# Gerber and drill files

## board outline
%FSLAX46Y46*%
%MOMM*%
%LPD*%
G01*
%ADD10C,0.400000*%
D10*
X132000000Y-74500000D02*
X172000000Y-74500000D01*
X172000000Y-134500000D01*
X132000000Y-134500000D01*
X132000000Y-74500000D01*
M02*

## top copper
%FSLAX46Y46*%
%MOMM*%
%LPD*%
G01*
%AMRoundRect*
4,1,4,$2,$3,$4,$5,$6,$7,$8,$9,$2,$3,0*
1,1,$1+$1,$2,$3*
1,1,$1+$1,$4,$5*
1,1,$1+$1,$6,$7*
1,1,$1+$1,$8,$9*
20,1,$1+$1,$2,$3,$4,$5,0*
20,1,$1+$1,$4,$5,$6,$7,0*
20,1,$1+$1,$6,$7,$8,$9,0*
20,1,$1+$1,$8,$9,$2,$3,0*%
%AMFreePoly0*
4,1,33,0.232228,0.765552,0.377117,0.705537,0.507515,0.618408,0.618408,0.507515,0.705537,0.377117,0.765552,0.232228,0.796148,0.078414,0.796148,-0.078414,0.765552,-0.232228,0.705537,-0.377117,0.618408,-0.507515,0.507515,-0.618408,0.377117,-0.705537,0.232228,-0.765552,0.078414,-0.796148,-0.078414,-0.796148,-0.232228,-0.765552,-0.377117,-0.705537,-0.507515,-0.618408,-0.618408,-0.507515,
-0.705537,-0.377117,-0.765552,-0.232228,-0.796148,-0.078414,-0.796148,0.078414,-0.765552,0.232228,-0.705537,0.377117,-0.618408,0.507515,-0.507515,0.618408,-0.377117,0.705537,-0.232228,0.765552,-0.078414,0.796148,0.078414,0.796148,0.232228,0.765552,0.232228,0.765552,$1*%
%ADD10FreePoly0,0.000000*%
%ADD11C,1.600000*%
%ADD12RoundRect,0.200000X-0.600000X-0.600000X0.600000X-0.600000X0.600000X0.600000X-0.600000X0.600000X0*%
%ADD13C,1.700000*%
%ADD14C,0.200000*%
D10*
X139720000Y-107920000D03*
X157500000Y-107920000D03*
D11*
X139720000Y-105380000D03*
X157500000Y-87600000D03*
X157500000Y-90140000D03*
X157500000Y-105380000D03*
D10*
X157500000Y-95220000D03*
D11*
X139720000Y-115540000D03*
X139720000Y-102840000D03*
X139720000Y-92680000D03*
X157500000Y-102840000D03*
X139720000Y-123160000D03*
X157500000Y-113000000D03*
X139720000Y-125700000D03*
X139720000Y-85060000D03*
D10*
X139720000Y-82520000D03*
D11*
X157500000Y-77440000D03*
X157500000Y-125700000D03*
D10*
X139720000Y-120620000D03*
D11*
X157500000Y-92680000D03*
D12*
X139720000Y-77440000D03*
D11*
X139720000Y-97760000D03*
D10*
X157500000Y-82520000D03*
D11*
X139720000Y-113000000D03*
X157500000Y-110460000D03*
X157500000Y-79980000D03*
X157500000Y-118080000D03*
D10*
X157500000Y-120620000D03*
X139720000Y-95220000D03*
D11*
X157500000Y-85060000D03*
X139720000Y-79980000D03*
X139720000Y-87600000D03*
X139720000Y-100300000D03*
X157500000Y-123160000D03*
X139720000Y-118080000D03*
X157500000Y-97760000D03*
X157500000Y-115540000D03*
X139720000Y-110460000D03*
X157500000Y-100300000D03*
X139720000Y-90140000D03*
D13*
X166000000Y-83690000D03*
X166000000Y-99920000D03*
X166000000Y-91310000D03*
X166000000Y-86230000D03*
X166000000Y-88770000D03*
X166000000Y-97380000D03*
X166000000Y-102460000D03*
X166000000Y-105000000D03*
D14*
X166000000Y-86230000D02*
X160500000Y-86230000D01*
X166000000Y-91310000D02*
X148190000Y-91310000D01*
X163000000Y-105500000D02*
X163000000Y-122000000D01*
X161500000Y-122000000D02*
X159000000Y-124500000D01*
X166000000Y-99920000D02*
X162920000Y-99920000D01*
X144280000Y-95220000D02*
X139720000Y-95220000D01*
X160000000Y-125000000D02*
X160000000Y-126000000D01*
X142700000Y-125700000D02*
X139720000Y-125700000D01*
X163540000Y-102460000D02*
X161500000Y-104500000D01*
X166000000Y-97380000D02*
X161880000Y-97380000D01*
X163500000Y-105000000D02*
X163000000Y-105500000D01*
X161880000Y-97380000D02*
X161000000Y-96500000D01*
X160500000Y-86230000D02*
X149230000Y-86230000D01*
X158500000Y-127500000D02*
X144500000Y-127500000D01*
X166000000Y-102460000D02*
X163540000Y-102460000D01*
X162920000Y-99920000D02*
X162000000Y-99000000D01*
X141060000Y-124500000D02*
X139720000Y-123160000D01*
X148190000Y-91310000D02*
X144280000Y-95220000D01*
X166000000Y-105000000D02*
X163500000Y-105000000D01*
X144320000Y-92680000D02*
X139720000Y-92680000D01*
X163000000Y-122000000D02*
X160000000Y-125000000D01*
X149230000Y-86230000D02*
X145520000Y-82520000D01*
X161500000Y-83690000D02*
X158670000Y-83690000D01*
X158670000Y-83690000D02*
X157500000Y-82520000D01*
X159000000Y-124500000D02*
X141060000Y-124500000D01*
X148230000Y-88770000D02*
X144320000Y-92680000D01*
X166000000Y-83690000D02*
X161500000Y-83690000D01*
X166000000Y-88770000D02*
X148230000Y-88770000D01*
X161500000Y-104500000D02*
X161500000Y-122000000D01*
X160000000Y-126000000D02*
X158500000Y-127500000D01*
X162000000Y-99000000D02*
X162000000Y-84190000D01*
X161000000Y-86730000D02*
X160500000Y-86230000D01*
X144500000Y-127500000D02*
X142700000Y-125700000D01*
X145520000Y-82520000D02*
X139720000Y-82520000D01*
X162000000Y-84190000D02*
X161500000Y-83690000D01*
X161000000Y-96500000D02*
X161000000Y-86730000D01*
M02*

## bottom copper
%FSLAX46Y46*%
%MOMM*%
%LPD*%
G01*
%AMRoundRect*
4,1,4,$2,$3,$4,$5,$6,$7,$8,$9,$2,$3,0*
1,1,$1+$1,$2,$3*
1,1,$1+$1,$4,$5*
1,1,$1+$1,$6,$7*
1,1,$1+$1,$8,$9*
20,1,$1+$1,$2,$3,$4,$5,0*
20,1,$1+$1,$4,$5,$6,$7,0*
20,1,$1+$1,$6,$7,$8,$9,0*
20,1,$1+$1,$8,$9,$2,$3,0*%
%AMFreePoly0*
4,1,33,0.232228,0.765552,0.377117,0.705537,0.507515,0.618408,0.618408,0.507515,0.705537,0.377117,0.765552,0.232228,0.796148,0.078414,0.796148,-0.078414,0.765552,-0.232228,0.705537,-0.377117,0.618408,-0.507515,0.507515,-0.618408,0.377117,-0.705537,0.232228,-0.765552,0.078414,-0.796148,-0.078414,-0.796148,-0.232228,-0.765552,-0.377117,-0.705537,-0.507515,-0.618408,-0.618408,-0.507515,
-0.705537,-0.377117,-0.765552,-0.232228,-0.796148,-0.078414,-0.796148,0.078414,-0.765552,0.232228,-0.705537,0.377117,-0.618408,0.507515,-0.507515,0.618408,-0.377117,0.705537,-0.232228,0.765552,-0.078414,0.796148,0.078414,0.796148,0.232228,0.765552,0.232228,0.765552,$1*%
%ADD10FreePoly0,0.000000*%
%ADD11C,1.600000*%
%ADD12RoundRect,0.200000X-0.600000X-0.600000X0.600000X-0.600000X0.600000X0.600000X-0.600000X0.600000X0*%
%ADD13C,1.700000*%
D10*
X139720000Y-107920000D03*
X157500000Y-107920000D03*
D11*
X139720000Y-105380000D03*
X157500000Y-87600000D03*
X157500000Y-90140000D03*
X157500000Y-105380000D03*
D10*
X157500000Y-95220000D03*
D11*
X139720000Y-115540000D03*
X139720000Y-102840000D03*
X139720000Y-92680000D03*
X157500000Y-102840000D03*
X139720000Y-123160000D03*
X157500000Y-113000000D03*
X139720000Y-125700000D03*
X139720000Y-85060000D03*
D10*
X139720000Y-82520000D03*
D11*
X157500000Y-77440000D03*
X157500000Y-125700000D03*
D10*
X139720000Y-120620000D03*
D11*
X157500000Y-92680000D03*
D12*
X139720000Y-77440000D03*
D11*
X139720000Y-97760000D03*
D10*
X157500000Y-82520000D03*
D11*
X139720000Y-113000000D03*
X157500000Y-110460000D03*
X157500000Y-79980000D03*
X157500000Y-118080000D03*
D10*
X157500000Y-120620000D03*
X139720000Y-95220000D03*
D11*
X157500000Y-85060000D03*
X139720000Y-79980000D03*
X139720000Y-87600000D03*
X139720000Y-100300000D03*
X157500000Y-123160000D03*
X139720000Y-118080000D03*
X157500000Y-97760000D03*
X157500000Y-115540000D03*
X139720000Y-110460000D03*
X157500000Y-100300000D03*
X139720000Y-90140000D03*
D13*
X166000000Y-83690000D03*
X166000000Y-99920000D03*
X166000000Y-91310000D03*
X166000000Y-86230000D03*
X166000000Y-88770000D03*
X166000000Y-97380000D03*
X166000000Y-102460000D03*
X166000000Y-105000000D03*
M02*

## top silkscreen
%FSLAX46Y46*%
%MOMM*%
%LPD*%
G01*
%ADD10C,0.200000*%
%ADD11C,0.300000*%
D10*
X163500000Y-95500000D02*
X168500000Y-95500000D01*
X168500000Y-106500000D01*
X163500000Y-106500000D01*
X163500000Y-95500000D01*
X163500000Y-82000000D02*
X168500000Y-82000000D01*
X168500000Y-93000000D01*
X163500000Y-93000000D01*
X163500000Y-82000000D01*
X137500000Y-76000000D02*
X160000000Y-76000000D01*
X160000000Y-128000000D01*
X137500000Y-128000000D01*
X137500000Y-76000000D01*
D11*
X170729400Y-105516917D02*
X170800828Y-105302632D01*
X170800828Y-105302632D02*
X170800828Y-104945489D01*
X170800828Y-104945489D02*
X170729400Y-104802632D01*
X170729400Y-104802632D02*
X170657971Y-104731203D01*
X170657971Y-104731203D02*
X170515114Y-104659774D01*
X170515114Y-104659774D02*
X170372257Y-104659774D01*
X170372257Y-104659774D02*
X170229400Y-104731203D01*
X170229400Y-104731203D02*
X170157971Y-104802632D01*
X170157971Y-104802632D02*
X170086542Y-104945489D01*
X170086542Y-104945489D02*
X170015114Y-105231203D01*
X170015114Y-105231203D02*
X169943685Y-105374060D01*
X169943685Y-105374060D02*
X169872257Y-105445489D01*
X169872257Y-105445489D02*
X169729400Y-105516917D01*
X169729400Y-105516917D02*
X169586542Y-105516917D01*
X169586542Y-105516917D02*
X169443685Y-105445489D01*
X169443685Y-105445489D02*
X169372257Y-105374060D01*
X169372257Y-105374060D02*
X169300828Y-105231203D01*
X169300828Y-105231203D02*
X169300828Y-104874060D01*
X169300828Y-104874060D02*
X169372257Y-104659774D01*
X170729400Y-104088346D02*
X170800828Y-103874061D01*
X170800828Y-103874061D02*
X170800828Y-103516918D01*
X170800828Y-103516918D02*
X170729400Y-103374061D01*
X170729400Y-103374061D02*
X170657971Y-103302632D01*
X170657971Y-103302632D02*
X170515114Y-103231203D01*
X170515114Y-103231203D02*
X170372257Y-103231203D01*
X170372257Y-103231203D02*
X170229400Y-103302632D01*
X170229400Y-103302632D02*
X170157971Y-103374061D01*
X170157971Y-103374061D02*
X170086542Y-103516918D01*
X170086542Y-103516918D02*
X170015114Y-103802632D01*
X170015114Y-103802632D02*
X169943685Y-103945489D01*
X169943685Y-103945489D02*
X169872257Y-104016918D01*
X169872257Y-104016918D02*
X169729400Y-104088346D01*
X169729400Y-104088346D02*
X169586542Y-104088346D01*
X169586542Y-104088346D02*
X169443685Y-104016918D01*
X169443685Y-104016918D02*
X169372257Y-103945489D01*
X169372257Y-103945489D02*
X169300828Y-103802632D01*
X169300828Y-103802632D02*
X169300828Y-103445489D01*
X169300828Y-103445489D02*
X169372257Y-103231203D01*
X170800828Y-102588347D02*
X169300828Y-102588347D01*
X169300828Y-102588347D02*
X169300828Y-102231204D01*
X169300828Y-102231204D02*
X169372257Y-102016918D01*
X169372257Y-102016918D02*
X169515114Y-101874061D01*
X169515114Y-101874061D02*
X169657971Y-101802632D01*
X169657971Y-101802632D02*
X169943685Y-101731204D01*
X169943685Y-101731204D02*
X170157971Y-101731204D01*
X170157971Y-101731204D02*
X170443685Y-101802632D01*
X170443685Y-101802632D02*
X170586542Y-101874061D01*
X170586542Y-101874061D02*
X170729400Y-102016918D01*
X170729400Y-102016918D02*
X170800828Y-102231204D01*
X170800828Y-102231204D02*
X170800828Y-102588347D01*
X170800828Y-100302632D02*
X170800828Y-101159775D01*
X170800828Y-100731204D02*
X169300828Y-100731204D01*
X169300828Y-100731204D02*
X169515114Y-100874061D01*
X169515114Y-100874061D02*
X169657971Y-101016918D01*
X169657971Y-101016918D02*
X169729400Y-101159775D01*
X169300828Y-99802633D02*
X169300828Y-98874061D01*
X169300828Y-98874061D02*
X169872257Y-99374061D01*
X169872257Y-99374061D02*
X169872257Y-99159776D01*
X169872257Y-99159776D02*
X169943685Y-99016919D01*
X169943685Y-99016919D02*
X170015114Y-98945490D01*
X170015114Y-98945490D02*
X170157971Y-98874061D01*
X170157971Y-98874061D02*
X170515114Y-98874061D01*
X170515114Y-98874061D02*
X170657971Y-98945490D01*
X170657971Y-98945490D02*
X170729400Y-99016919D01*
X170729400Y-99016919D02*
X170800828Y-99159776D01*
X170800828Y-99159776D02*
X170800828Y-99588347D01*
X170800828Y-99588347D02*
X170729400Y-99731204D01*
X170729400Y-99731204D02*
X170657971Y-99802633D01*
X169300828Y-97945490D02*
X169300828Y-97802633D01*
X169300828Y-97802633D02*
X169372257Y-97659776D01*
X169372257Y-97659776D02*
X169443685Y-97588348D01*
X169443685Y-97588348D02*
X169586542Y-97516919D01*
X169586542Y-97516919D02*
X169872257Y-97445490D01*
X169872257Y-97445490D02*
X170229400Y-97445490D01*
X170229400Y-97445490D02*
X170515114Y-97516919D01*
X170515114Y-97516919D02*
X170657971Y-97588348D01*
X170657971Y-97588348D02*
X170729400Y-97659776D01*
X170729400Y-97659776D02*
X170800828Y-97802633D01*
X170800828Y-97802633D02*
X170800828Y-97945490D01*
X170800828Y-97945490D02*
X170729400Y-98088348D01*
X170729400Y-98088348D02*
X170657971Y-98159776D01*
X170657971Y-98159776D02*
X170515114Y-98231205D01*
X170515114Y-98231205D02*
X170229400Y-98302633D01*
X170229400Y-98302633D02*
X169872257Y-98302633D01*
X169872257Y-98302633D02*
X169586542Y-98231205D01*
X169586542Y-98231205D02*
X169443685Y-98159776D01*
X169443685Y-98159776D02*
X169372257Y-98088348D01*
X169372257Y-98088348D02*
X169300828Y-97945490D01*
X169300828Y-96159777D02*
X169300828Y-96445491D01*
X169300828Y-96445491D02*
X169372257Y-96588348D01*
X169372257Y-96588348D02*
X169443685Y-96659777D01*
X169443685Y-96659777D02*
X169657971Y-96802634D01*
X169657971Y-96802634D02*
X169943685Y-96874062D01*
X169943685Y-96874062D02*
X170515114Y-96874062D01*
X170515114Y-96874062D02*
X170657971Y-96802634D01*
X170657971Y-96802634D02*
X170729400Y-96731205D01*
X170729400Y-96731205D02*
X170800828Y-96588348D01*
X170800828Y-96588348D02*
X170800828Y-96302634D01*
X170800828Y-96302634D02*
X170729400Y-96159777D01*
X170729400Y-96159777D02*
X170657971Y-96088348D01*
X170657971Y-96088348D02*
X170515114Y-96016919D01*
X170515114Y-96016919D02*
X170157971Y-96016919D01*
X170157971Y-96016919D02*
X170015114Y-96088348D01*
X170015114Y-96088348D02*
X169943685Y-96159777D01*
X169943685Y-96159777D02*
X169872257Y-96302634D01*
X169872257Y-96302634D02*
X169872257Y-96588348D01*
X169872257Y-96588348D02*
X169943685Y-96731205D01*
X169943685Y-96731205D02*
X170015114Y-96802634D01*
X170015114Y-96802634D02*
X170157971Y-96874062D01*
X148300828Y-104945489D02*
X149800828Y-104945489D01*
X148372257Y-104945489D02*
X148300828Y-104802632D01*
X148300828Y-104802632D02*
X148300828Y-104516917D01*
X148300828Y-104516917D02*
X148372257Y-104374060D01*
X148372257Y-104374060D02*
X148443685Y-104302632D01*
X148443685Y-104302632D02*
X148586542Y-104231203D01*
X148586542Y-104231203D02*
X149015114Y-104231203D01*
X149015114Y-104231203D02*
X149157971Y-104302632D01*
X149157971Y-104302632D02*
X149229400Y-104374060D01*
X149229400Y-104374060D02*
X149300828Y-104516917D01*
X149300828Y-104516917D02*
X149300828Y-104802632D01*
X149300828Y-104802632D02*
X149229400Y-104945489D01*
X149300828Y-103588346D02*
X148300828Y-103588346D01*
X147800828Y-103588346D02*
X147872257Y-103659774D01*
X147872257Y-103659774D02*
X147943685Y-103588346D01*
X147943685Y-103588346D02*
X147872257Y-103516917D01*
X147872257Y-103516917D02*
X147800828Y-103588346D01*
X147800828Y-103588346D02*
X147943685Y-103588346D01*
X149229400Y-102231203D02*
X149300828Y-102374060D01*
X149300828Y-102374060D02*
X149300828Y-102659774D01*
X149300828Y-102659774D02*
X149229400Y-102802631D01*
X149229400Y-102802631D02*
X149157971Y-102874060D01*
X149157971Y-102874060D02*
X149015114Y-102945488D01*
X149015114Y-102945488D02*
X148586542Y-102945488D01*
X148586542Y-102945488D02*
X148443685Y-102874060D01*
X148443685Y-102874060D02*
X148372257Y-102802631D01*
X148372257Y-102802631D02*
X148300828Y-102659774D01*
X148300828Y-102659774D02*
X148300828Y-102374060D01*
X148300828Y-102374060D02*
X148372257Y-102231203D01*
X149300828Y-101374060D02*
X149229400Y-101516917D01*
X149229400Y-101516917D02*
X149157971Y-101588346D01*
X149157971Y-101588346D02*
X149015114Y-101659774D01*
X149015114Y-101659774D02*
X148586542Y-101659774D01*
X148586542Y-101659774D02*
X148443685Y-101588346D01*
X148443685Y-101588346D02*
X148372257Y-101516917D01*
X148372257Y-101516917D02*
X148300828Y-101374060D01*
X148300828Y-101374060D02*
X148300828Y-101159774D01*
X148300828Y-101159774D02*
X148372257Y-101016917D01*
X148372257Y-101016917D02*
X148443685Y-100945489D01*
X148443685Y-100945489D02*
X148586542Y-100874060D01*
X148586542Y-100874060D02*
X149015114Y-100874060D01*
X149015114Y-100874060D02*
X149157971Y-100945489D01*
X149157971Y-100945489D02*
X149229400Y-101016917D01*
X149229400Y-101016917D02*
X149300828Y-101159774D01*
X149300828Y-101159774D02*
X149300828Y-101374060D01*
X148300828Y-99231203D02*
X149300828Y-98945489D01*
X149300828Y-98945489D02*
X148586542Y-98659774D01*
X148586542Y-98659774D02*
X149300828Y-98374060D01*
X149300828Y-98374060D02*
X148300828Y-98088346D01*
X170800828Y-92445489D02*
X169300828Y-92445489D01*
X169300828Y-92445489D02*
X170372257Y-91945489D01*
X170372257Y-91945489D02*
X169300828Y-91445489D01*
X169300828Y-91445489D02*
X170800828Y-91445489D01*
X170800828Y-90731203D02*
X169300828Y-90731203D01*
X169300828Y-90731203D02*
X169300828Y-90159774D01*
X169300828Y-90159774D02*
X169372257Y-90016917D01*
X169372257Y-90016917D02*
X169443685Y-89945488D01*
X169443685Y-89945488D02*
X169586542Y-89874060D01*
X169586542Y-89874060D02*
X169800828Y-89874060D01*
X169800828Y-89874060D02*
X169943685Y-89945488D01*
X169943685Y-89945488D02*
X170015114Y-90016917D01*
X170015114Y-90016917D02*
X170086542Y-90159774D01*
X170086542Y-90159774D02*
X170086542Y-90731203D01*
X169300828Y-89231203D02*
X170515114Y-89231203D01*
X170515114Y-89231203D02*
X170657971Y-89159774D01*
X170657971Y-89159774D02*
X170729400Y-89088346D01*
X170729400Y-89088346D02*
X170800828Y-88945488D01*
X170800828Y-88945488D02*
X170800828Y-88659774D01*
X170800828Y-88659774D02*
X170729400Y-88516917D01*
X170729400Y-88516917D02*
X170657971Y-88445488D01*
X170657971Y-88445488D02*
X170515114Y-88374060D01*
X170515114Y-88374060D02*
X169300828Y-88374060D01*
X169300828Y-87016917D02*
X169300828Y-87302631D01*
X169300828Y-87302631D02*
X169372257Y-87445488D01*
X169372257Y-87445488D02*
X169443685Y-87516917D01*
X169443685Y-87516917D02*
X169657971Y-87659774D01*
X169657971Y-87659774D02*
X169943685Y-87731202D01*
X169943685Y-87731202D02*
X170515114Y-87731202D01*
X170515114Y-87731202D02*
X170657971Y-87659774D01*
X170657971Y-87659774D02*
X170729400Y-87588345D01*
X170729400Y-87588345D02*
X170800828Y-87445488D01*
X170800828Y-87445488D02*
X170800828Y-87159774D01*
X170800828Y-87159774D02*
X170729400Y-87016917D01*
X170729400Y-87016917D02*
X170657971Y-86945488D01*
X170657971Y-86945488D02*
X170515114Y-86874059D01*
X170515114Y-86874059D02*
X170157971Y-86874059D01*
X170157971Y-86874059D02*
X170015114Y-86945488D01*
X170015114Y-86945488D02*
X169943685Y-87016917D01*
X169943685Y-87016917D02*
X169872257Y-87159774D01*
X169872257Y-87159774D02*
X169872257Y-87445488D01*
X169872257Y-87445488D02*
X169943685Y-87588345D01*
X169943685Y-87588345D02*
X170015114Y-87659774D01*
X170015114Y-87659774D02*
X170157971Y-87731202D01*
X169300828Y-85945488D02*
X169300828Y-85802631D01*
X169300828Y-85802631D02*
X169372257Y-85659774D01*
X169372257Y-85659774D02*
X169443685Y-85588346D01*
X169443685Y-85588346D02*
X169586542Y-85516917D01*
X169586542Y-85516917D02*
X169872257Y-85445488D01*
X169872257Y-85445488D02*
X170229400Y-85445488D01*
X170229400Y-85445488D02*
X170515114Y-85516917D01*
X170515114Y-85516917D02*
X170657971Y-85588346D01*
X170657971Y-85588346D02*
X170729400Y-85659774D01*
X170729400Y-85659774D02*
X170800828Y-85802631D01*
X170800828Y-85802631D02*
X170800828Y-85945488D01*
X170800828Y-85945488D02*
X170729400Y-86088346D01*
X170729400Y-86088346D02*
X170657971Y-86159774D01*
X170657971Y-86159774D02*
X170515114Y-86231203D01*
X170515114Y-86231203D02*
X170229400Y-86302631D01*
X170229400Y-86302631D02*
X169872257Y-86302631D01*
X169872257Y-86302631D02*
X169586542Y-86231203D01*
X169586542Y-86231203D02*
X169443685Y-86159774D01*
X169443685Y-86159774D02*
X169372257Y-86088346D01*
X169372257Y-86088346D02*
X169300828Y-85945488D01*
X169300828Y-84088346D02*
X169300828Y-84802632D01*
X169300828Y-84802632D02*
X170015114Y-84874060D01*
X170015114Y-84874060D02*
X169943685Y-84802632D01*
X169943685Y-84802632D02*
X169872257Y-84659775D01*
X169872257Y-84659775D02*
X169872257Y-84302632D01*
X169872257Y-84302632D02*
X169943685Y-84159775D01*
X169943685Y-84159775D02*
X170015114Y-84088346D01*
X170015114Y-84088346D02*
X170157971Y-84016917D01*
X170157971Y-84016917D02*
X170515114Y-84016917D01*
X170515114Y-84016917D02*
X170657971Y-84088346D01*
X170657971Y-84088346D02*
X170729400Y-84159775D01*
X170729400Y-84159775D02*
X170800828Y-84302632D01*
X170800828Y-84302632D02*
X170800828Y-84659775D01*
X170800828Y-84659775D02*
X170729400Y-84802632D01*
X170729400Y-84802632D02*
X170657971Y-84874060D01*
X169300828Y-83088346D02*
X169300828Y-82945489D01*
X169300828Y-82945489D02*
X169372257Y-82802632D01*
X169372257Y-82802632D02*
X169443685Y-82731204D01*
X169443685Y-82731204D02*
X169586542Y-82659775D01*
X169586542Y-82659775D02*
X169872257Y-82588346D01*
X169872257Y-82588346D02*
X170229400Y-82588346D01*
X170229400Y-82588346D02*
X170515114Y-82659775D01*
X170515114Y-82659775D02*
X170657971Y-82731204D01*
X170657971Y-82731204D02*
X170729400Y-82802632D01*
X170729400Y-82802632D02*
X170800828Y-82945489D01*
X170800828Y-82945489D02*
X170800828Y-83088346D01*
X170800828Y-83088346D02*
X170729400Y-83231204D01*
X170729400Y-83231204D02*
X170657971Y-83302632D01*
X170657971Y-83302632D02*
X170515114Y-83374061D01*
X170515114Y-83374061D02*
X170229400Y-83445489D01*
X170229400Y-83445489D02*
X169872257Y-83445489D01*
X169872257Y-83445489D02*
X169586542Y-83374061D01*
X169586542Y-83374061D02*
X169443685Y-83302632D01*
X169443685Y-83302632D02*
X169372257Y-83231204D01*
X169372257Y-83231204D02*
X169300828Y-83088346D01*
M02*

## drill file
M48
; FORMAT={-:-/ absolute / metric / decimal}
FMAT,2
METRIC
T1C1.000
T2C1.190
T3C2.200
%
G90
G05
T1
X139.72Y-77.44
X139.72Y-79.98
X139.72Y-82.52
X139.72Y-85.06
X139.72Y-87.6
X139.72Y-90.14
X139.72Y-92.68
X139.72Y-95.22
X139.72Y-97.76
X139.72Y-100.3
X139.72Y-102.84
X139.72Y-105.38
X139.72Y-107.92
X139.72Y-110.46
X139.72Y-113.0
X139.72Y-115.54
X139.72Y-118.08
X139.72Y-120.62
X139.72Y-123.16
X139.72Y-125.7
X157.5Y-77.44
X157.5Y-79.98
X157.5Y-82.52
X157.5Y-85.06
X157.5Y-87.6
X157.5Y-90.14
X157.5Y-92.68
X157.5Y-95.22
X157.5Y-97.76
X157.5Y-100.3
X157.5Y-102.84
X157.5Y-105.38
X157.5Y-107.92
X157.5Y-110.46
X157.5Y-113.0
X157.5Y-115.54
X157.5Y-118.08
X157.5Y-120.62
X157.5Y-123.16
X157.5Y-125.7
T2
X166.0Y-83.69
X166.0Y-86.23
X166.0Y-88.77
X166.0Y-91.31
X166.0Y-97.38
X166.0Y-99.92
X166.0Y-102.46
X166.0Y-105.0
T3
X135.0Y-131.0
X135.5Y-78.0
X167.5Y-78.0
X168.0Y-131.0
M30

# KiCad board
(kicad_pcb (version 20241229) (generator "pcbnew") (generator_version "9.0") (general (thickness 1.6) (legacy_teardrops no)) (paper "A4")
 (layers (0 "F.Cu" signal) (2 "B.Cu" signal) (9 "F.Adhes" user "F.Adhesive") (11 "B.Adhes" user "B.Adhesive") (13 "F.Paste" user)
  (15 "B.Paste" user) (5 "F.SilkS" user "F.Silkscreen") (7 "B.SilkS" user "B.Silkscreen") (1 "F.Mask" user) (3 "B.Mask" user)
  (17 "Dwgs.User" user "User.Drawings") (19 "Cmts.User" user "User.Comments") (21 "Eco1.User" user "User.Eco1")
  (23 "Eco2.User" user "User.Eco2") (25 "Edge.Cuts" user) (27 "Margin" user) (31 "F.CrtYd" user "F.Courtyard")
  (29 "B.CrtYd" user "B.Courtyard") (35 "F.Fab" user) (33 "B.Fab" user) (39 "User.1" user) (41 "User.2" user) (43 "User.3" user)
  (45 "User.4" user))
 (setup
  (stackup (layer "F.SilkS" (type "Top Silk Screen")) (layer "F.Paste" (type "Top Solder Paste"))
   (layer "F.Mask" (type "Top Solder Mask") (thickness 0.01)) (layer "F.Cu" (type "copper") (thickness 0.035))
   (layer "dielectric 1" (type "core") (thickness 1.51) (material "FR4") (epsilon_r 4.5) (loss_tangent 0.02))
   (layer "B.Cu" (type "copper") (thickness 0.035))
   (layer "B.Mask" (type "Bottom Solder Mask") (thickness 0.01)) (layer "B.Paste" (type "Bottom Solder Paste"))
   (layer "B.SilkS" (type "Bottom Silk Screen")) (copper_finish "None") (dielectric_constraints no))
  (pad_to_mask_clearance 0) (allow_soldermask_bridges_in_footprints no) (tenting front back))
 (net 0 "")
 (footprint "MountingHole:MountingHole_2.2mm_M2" (layer "F.Cu") (at 135 131)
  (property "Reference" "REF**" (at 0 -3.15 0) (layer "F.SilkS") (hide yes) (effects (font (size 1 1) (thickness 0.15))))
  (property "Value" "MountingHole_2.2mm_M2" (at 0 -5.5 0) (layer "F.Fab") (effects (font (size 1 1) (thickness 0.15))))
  (pad "" np_thru_hole circle (at 0 0) (size 2.2 2.2) (drill 2.2) (layers "*.Cu" "*.Mask")))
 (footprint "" (layer "F.Cu") (at 139.72 107.92)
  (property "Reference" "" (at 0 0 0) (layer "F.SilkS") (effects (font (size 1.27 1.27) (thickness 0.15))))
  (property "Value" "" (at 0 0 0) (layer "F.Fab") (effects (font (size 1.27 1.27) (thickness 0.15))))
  (pad "13" thru_hole custom (at 0 0) (size 1.6 1.6) (drill 1) (layers "*.Cu" "*.Mask") (remove_unused_layers no)
   (options (clearance outline) (anchor circle)) (primitives)))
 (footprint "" (layer "F.Cu") (at 157.5 107.92)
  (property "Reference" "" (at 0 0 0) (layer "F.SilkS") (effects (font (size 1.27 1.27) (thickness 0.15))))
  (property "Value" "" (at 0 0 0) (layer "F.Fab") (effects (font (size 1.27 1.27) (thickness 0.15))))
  (pad "28" thru_hole custom (at 0 0) (size 1.6 1.6) (drill 1) (layers "*.Cu" "*.Mask") (remove_unused_layers no)
   (options (clearance outline) (anchor circle)) (primitives)))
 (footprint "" (layer "F.Cu") (at 139.72 105.38)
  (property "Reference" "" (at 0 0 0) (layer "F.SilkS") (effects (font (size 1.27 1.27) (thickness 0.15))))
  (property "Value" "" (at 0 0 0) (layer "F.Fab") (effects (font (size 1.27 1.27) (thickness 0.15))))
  (pad "12" thru_hole circle (at 0 0) (size 1.6 1.6) (drill 1) (layers "*.Cu" "*.Mask") (remove_unused_layers no)))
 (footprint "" (layer "F.Cu") (at 157.5 87.6)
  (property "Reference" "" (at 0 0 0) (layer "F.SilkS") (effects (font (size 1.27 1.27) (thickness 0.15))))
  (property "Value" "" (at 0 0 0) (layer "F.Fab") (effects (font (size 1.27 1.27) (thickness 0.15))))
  (pad "36" thru_hole circle (at 0 0) (size 1.6 1.6) (drill 1) (layers "*.Cu" "*.Mask") (remove_unused_layers no)))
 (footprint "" (layer "F.Cu") (at 157.5 90.14)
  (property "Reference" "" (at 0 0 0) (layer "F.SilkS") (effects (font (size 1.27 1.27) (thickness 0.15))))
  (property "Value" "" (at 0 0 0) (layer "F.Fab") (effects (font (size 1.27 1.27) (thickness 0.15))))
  (pad "35" thru_hole circle (at 0 0) (size 1.6 1.6) (drill 1) (layers "*.Cu" "*.Mask") (remove_unused_layers no)))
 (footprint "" (layer "F.Cu") (at 157.5 105.38)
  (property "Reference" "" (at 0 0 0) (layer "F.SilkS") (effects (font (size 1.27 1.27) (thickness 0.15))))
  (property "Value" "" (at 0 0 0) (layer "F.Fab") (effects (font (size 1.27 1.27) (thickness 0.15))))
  (pad "29" thru_hole circle (at 0 0) (size 1.6 1.6) (drill 1) (layers "*.Cu" "*.Mask") (remove_unused_layers no)))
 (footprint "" (layer "F.Cu") (at 157.5 95.22)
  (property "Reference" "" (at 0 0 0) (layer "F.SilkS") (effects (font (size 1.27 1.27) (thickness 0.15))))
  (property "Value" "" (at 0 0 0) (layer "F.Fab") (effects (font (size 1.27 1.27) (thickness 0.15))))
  (pad "33" thru_hole custom (at 0 0) (size 1.6 1.6) (drill 1) (layers "*.Cu" "*.Mask") (remove_unused_layers no)
   (options (clearance outline) (anchor circle)) (primitives)))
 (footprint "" (layer "F.Cu") (at 139.72 115.54)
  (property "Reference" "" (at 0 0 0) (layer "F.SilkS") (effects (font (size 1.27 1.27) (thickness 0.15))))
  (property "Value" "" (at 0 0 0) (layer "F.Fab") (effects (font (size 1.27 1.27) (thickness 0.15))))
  (pad "16" thru_hole circle (at 0 0) (size 1.6 1.6) (drill 1) (layers "*.Cu" "*.Mask") (remove_unused_layers no)))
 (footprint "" (layer "F.Cu") (at 139.72 102.84)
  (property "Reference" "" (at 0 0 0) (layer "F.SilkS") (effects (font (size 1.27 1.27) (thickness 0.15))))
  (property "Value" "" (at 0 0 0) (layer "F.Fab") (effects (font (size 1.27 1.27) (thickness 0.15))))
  (pad "11" thru_hole circle (at 0 0) (size 1.6 1.6) (drill 1) (layers "*.Cu" "*.Mask") (remove_unused_layers no)))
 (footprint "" (layer "F.Cu") (at 139.72 92.68)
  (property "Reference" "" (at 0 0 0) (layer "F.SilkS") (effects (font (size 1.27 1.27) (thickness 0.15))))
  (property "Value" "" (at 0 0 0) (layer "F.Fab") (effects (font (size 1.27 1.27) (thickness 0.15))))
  (pad "7" thru_hole circle (at 0 0) (size 1.6 1.6) (drill 1) (layers "*.Cu" "*.Mask") (remove_unused_layers no)))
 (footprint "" (layer "F.Cu") (at 157.5 102.84)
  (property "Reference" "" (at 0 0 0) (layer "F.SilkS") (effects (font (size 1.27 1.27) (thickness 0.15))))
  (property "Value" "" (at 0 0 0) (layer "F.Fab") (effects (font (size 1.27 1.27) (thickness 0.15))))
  (pad "30" thru_hole circle (at 0 0) (size 1.6 1.6) (drill 1) (layers "*.Cu" "*.Mask") (remove_unused_layers no)))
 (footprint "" (layer "F.Cu") (at 139.72 123.16)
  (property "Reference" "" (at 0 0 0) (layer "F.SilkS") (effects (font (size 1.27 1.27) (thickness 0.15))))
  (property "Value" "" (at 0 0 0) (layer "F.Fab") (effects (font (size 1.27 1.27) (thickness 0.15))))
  (pad "19" thru_hole circle (at 0 0) (size 1.6 1.6) (drill 1) (layers "*.Cu" "*.Mask") (remove_unused_layers no)))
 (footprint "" (layer "F.Cu") (at 157.5 113)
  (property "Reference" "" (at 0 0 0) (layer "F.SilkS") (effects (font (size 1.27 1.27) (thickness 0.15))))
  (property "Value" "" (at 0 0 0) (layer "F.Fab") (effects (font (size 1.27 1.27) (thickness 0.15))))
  (pad "26" thru_hole circle (at 0 0) (size 1.6 1.6) (drill 1) (layers "*.Cu" "*.Mask") (remove_unused_layers no)))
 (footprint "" (layer "F.Cu") (at 139.72 125.7)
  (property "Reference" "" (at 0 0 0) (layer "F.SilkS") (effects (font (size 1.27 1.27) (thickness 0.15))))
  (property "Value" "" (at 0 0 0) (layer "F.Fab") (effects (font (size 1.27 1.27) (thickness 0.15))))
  (pad "20" thru_hole circle (at 0 0) (size 1.6 1.6) (drill 1) (layers "*.Cu" "*.Mask") (remove_unused_layers no)))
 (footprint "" (layer "F.Cu") (at 139.72 85.06)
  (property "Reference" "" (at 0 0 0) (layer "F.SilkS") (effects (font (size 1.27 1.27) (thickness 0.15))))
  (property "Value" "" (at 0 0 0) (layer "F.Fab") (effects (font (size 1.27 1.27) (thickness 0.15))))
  (pad "4" thru_hole circle (at 0 0) (size 1.6 1.6) (drill 1) (layers "*.Cu" "*.Mask") (remove_unused_layers no)))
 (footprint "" (layer "F.Cu") (at 139.72 82.52)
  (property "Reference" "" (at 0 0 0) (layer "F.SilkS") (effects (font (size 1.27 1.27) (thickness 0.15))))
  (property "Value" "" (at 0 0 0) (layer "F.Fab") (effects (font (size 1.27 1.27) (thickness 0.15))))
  (pad "3" thru_hole custom (at 0 0) (size 1.6 1.6) (drill 1) (layers "*.Cu" "*.Mask") (remove_unused_layers no)
   (options (clearance outline) (anchor circle)) (primitives)))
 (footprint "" (layer "F.Cu") (at 157.5 77.44)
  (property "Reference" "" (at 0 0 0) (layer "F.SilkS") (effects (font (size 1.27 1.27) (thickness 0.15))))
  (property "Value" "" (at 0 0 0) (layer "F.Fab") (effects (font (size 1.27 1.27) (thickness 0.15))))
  (pad "40" thru_hole circle (at 0 0) (size 1.6 1.6) (drill 1) (layers "*.Cu" "*.Mask") (remove_unused_layers no)))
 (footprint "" (layer "F.Cu") (at 157.5 125.7)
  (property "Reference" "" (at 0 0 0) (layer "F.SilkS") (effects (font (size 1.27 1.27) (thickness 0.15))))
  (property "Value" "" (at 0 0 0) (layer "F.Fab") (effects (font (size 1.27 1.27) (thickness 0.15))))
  (pad "21" thru_hole circle (at 0 0) (size 1.6 1.6) (drill 1) (layers "*.Cu" "*.Mask") (remove_unused_layers no)))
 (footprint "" (layer "F.Cu") (at 139.72 120.62)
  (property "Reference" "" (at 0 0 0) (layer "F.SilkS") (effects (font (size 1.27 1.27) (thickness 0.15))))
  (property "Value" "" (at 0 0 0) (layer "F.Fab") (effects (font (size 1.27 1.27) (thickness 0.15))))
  (pad "18" thru_hole custom (at 0 0) (size 1.6 1.6) (drill 1) (layers "*.Cu" "*.Mask") (remove_unused_layers no)
   (options (clearance outline) (anchor circle)) (primitives)))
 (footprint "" (layer "F.Cu") (at 157.5 92.68)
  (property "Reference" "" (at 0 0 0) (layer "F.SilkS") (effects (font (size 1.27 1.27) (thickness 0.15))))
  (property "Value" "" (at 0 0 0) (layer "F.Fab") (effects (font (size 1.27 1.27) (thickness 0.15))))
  (pad "34" thru_hole circle (at 0 0) (size 1.6 1.6) (drill 1) (layers "*.Cu" "*.Mask") (remove_unused_layers no)))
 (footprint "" (layer "F.Cu") (at 139.72 77.44)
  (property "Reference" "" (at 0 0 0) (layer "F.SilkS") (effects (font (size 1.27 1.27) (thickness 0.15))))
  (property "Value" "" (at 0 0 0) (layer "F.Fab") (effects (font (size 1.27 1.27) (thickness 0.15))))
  (pad "1" thru_hole roundrect (at 0 0) (size 1.6 1.6) (drill 1) (layers "*.Cu" "*.Mask") (remove_unused_layers no) (roundrect_rratio 0.125)))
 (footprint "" (layer "F.Cu") (at 139.72 97.76)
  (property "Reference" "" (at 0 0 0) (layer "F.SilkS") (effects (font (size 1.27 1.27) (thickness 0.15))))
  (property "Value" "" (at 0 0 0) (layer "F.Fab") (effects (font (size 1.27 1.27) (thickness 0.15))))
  (pad "9" thru_hole circle (at 0 0) (size 1.6 1.6) (drill 1) (layers "*.Cu" "*.Mask") (remove_unused_layers no)))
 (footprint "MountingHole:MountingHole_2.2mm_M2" (layer "F.Cu") (at 168 131)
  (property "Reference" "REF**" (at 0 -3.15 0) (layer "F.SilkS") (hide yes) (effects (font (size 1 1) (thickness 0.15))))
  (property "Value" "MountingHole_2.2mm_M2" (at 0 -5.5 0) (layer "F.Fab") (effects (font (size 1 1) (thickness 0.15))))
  (pad "" np_thru_hole circle (at 0 0) (size 2.2 2.2) (drill 2.2) (layers "*.Cu" "*.Mask")))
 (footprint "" (layer "F.Cu") (at 157.5 82.52)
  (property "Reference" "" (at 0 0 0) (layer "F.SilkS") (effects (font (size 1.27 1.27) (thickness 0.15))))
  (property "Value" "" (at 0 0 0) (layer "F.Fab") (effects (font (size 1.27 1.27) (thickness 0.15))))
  (pad "38" thru_hole custom (at 0 0) (size 1.6 1.6) (drill 1) (layers "*.Cu" "*.Mask") (remove_unused_layers no)
   (options (clearance outline) (anchor circle)) (primitives)))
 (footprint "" (layer "F.Cu") (at 139.72 113)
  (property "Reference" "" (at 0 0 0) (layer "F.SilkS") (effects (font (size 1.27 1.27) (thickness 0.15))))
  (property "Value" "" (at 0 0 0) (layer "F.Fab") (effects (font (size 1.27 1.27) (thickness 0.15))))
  (pad "15" thru_hole circle (at 0 0) (size 1.6 1.6) (drill 1) (layers "*.Cu" "*.Mask") (remove_unused_layers no)))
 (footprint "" (layer "F.Cu") (at 157.5 110.46)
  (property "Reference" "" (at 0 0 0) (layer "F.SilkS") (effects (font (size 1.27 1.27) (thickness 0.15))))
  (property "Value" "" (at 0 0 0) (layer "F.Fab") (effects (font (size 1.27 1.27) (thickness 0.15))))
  (pad "27" thru_hole circle (at 0 0) (size 1.6 1.6) (drill 1) (layers "*.Cu" "*.Mask") (remove_unused_layers no)))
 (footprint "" (layer "F.Cu") (at 157.5 79.98)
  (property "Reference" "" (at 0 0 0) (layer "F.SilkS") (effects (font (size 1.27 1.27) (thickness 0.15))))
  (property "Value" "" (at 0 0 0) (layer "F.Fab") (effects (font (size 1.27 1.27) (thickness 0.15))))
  (pad "39" thru_hole circle (at 0 0) (size 1.6 1.6) (drill 1) (layers "*.Cu" "*.Mask") (remove_unused_layers no)))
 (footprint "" (layer "F.Cu") (at 157.5 118.08)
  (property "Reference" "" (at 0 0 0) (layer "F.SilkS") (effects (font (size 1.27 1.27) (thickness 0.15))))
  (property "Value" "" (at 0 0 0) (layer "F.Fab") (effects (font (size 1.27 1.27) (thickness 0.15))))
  (pad "24" thru_hole circle (at 0 0) (size 1.6 1.6) (drill 1) (layers "*.Cu" "*.Mask") (remove_unused_layers no)))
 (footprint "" (layer "F.Cu") (at 157.5 120.62)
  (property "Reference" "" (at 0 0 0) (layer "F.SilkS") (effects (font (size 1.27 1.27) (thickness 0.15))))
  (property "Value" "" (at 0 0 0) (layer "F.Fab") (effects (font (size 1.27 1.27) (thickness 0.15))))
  (pad "23" thru_hole custom (at 0 0) (size 1.6 1.6) (drill 1) (layers "*.Cu" "*.Mask") (remove_unused_layers no)
   (options (clearance outline) (anchor circle)) (primitives)))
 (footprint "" (layer "F.Cu") (at 139.72 95.22)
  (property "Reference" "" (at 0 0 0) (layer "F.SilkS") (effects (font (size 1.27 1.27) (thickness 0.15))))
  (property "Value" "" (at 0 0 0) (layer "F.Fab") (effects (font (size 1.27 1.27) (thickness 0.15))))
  (pad "8" thru_hole custom (at 0 0) (size 1.6 1.6) (drill 1) (layers "*.Cu" "*.Mask") (remove_unused_layers no)
   (options (clearance outline) (anchor circle)) (primitives)))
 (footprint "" (layer "F.Cu") (at 157.5 85.06)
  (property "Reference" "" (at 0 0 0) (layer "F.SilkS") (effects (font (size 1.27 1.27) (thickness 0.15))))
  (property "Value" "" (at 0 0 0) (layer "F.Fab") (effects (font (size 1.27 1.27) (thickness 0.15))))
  (pad "37" thru_hole circle (at 0 0) (size 1.6 1.6) (drill 1) (layers "*.Cu" "*.Mask") (remove_unused_layers no)))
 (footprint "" (layer "F.Cu") (at 139.72 79.98)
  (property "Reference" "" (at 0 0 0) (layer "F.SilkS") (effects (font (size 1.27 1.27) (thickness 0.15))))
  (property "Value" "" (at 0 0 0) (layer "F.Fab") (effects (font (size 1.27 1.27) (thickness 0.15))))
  (pad "2" thru_hole circle (at 0 0) (size 1.6 1.6) (drill 1) (layers "*.Cu" "*.Mask") (remove_unused_layers no)))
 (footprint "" (layer "F.Cu") (at 139.72 87.6)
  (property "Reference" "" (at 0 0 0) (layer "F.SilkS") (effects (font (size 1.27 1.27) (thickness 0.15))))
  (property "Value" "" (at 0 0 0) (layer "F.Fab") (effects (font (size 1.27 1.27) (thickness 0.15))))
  (pad "5" thru_hole circle (at 0 0) (size 1.6 1.6) (drill 1) (layers "*.Cu" "*.Mask") (remove_unused_layers no)))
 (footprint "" (layer "F.Cu") (at 139.72 100.3)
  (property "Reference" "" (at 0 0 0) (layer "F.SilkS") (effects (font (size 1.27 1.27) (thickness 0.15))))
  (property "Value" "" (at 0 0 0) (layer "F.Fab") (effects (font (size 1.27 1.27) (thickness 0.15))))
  (pad "10" thru_hole circle (at 0 0) (size 1.6 1.6) (drill 1) (layers "*.Cu" "*.Mask") (remove_unused_layers no)))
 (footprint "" (layer "F.Cu") (at 157.5 123.16)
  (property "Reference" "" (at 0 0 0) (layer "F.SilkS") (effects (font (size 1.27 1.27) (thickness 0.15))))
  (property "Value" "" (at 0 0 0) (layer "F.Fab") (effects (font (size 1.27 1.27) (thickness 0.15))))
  (pad "22" thru_hole circle (at 0 0) (size 1.6 1.6) (drill 1) (layers "*.Cu" "*.Mask") (remove_unused_layers no)))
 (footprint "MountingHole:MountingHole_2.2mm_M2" (layer "F.Cu") (at 167.5 78)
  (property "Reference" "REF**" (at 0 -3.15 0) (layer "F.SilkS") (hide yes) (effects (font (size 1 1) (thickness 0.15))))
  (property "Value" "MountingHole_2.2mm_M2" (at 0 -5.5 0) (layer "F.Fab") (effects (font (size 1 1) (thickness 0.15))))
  (pad "" np_thru_hole circle (at 0 0) (size 2.2 2.2) (drill 2.2) (layers "*.Cu" "*.Mask")))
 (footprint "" (layer "F.Cu") (at 139.72 118.08)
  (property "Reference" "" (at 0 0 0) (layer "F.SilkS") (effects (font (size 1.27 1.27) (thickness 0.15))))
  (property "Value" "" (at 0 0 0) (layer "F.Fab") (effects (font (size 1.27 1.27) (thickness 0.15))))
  (pad "17" thru_hole circle (at 0 0) (size 1.6 1.6) (drill 1) (layers "*.Cu" "*.Mask") (remove_unused_layers no)))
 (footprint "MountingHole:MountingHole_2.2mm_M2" (layer "F.Cu") (at 135.5 78)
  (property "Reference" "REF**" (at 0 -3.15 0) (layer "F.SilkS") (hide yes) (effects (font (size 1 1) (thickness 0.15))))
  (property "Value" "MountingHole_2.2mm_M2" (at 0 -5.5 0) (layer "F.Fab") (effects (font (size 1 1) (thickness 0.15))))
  (pad "" np_thru_hole circle (at 0 0) (size 2.2 2.2) (drill 2.2) (layers "*.Cu" "*.Mask")))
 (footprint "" (layer "F.Cu") (at 157.5 97.76)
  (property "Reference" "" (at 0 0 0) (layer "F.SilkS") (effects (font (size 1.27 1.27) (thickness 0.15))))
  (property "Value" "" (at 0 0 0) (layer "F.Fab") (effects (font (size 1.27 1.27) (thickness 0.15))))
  (pad "32" thru_hole circle (at 0 0) (size 1.6 1.6) (drill 1) (layers "*.Cu" "*.Mask") (remove_unused_layers no)))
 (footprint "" (layer "F.Cu") (at 157.5 115.54)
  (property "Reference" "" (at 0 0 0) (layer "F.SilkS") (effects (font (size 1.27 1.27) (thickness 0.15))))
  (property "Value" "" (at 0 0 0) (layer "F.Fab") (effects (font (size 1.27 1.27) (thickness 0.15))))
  (pad "25" thru_hole circle (at 0 0) (size 1.6 1.6) (drill 1) (layers "*.Cu" "*.Mask") (remove_unused_layers no)))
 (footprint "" (layer "F.Cu") (at 139.72 110.46)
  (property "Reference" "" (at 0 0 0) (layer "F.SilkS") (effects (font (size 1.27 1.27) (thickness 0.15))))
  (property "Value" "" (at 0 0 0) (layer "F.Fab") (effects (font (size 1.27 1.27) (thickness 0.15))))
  (pad "14" thru_hole circle (at 0 0) (size 1.6 1.6) (drill 1) (layers "*.Cu" "*.Mask") (remove_unused_layers no)))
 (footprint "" (layer "F.Cu") (at 157.5 100.3)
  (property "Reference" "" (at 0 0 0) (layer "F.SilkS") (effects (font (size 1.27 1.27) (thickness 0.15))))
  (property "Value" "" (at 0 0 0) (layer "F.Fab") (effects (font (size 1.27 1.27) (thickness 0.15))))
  (pad "31" thru_hole circle (at 0 0) (size 1.6 1.6) (drill 1) (layers "*.Cu" "*.Mask") (remove_unused_layers no)))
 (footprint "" (layer "F.Cu") (at 139.72 90.14)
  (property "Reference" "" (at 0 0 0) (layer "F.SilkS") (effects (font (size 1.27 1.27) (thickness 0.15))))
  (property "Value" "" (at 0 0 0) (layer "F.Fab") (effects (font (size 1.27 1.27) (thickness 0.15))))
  (pad "6" thru_hole circle (at 0 0) (size 1.6 1.6) (drill 1) (layers "*.Cu" "*.Mask") (remove_unused_layers no)))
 (gr_rect (start 163.5 95.5) (end 168.5 106.5) (stroke (width 0.2) (type solid)) (fill no) (layer "F.SilkS"))
 (gr_rect (start 163.5 82) (end 168.5 93) (stroke (width 0.2) (type solid)) (fill no) (layer "F.SilkS"))
 (gr_rect (start 137.5 76) (end 160 128) (stroke (width 0.2) (type solid)) (fill no) (layer "F.SilkS"))
 (gr_rect (start 132 74.5) (end 172 134.5) (stroke (width 0.4) (type solid)) (fill no) (layer "Edge.Cuts"))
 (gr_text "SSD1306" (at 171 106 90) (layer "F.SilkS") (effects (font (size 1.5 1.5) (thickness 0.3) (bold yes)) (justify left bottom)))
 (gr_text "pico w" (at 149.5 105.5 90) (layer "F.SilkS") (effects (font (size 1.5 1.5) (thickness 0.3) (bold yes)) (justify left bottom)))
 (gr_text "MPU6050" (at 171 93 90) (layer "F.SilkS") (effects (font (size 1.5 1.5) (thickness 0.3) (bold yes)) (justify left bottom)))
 (segment (start 166 86.23) (end 160.5 86.23) (width 0.2) (layer "F.Cu") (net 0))
 (segment (start 166 91.31) (end 148.19 91.31) (width 0.2) (layer "F.Cu") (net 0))
 (segment (start 163 105.5) (end 163 122) (width 0.2) (layer "F.Cu") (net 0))
 (segment (start 161.5 122) (end 159 124.5) (width 0.2) (layer "F.Cu") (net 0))
 (segment (start 166 99.92) (end 162.92 99.92) (width 0.2) (layer "F.Cu") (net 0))
 (segment (start 144.28 95.22) (end 139.72 95.22) (width 0.2) (layer "F.Cu") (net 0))
 (segment (start 160 125) (end 160 126) (width 0.2) (layer "F.Cu") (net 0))
 (segment (start 142.7 125.7) (end 139.72 125.7) (width 0.2) (layer "F.Cu") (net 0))
 (segment (start 163.54 102.46) (end 161.5 104.5) (width 0.2) (layer "F.Cu") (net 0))
 (segment (start 166 97.38) (end 161.88 97.38) (width 0.2) (layer "F.Cu") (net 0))
 (segment (start 163.5 105) (end 163 105.5) (width 0.2) (layer "F.Cu") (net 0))
 (segment (start 161.88 97.38) (end 161 96.5) (width 0.2) (layer "F.Cu") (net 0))
 (segment (start 160.5 86.23) (end 149.23 86.23) (width 0.2) (layer "F.Cu") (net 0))
 (segment (start 158.5 127.5) (end 144.5 127.5) (width 0.2) (layer "F.Cu") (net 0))
 (segment (start 166 102.46) (end 163.54 102.46) (width 0.2) (layer "F.Cu") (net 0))
 (segment (start 162.92 99.92) (end 162 99) (width 0.2) (layer "F.Cu") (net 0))
 (segment (start 141.06 124.5) (end 139.72 123.16) (width 0.2) (layer "F.Cu") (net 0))
 (segment (start 148.19 91.31) (end 144.28 95.22) (width 0.2) (layer "F.Cu") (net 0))
 (segment (start 166 105) (end 163.5 105) (width 0.2) (layer "F.Cu") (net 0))
 (segment (start 144.32 92.68) (end 139.72 92.68) (width 0.2) (layer "F.Cu") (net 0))
 (segment (start 163 122) (end 160 125) (width 0.2) (layer "F.Cu") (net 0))
 (segment (start 149.23 86.23) (end 145.52 82.52) (width 0.2) (layer "F.Cu") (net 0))
 (segment (start 161.5 83.69) (end 158.67 83.69) (width 0.2) (layer "F.Cu") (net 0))
 (segment (start 158.67 83.69) (end 157.5 82.52) (width 0.2) (layer "F.Cu") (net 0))
 (segment (start 159 124.5) (end 141.06 124.5) (width 0.2) (layer "F.Cu") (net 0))
 (segment (start 148.23 88.77) (end 144.32 92.68) (width 0.2) (layer "F.Cu") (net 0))
 (segment (start 166 83.69) (end 161.5 83.69) (width 0.2) (layer "F.Cu") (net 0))
 (segment (start 166 88.77) (end 148.23 88.77) (width 0.2) (layer "F.Cu") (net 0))
 (segment (start 161.5 104.5) (end 161.5 122) (width 0.2) (layer "F.Cu") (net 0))
 (segment (start 160 126) (end 158.5 127.5) (width 0.2) (layer "F.Cu") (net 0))
 (segment (start 162 99) (end 162 84.19) (width 0.2) (layer "F.Cu") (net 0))
 (segment (start 161 86.73) (end 160.5 86.23) (width 0.2) (layer "F.Cu") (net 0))
 (segment (start 144.5 127.5) (end 142.7 125.7) (width 0.2) (layer "F.Cu") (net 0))
 (segment (start 145.52 82.52) (end 139.72 82.52) (width 0.2) (layer "F.Cu") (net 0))
 (segment (start 162 84.19) (end 161.5 83.69) (width 0.2) (layer "F.Cu") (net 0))
 (segment (start 161 96.5) (end 161 86.73) (width 0.2) (layer "F.Cu") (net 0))
 (via (at 166 83.69) (size 1.7) (drill 1.19) (layers "F.Cu" "B.Cu") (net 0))
 (via (at 166 99.92) (size 1.7) (drill 1.19) (layers "F.Cu" "B.Cu") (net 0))
 (via (at 166 91.31) (size 1.7) (drill 1.19) (layers "F.Cu" "B.Cu") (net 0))
 (via (at 166 86.23) (size 1.7) (drill 1.19) (layers "F.Cu" "B.Cu") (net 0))
 (via (at 166 88.77) (size 1.7) (drill 1.19) (layers "F.Cu" "B.Cu") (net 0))
 (via (at 166 97.38) (size 1.7) (drill 1.19) (layers "F.Cu" "B.Cu") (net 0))
 (via (at 166 102.46) (size 1.7) (drill 1.19) (layers "F.Cu" "B.Cu") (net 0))
 (via (at 166 105) (size 1.7) (drill 1.19) (layers "F.Cu" "B.Cu") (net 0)))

